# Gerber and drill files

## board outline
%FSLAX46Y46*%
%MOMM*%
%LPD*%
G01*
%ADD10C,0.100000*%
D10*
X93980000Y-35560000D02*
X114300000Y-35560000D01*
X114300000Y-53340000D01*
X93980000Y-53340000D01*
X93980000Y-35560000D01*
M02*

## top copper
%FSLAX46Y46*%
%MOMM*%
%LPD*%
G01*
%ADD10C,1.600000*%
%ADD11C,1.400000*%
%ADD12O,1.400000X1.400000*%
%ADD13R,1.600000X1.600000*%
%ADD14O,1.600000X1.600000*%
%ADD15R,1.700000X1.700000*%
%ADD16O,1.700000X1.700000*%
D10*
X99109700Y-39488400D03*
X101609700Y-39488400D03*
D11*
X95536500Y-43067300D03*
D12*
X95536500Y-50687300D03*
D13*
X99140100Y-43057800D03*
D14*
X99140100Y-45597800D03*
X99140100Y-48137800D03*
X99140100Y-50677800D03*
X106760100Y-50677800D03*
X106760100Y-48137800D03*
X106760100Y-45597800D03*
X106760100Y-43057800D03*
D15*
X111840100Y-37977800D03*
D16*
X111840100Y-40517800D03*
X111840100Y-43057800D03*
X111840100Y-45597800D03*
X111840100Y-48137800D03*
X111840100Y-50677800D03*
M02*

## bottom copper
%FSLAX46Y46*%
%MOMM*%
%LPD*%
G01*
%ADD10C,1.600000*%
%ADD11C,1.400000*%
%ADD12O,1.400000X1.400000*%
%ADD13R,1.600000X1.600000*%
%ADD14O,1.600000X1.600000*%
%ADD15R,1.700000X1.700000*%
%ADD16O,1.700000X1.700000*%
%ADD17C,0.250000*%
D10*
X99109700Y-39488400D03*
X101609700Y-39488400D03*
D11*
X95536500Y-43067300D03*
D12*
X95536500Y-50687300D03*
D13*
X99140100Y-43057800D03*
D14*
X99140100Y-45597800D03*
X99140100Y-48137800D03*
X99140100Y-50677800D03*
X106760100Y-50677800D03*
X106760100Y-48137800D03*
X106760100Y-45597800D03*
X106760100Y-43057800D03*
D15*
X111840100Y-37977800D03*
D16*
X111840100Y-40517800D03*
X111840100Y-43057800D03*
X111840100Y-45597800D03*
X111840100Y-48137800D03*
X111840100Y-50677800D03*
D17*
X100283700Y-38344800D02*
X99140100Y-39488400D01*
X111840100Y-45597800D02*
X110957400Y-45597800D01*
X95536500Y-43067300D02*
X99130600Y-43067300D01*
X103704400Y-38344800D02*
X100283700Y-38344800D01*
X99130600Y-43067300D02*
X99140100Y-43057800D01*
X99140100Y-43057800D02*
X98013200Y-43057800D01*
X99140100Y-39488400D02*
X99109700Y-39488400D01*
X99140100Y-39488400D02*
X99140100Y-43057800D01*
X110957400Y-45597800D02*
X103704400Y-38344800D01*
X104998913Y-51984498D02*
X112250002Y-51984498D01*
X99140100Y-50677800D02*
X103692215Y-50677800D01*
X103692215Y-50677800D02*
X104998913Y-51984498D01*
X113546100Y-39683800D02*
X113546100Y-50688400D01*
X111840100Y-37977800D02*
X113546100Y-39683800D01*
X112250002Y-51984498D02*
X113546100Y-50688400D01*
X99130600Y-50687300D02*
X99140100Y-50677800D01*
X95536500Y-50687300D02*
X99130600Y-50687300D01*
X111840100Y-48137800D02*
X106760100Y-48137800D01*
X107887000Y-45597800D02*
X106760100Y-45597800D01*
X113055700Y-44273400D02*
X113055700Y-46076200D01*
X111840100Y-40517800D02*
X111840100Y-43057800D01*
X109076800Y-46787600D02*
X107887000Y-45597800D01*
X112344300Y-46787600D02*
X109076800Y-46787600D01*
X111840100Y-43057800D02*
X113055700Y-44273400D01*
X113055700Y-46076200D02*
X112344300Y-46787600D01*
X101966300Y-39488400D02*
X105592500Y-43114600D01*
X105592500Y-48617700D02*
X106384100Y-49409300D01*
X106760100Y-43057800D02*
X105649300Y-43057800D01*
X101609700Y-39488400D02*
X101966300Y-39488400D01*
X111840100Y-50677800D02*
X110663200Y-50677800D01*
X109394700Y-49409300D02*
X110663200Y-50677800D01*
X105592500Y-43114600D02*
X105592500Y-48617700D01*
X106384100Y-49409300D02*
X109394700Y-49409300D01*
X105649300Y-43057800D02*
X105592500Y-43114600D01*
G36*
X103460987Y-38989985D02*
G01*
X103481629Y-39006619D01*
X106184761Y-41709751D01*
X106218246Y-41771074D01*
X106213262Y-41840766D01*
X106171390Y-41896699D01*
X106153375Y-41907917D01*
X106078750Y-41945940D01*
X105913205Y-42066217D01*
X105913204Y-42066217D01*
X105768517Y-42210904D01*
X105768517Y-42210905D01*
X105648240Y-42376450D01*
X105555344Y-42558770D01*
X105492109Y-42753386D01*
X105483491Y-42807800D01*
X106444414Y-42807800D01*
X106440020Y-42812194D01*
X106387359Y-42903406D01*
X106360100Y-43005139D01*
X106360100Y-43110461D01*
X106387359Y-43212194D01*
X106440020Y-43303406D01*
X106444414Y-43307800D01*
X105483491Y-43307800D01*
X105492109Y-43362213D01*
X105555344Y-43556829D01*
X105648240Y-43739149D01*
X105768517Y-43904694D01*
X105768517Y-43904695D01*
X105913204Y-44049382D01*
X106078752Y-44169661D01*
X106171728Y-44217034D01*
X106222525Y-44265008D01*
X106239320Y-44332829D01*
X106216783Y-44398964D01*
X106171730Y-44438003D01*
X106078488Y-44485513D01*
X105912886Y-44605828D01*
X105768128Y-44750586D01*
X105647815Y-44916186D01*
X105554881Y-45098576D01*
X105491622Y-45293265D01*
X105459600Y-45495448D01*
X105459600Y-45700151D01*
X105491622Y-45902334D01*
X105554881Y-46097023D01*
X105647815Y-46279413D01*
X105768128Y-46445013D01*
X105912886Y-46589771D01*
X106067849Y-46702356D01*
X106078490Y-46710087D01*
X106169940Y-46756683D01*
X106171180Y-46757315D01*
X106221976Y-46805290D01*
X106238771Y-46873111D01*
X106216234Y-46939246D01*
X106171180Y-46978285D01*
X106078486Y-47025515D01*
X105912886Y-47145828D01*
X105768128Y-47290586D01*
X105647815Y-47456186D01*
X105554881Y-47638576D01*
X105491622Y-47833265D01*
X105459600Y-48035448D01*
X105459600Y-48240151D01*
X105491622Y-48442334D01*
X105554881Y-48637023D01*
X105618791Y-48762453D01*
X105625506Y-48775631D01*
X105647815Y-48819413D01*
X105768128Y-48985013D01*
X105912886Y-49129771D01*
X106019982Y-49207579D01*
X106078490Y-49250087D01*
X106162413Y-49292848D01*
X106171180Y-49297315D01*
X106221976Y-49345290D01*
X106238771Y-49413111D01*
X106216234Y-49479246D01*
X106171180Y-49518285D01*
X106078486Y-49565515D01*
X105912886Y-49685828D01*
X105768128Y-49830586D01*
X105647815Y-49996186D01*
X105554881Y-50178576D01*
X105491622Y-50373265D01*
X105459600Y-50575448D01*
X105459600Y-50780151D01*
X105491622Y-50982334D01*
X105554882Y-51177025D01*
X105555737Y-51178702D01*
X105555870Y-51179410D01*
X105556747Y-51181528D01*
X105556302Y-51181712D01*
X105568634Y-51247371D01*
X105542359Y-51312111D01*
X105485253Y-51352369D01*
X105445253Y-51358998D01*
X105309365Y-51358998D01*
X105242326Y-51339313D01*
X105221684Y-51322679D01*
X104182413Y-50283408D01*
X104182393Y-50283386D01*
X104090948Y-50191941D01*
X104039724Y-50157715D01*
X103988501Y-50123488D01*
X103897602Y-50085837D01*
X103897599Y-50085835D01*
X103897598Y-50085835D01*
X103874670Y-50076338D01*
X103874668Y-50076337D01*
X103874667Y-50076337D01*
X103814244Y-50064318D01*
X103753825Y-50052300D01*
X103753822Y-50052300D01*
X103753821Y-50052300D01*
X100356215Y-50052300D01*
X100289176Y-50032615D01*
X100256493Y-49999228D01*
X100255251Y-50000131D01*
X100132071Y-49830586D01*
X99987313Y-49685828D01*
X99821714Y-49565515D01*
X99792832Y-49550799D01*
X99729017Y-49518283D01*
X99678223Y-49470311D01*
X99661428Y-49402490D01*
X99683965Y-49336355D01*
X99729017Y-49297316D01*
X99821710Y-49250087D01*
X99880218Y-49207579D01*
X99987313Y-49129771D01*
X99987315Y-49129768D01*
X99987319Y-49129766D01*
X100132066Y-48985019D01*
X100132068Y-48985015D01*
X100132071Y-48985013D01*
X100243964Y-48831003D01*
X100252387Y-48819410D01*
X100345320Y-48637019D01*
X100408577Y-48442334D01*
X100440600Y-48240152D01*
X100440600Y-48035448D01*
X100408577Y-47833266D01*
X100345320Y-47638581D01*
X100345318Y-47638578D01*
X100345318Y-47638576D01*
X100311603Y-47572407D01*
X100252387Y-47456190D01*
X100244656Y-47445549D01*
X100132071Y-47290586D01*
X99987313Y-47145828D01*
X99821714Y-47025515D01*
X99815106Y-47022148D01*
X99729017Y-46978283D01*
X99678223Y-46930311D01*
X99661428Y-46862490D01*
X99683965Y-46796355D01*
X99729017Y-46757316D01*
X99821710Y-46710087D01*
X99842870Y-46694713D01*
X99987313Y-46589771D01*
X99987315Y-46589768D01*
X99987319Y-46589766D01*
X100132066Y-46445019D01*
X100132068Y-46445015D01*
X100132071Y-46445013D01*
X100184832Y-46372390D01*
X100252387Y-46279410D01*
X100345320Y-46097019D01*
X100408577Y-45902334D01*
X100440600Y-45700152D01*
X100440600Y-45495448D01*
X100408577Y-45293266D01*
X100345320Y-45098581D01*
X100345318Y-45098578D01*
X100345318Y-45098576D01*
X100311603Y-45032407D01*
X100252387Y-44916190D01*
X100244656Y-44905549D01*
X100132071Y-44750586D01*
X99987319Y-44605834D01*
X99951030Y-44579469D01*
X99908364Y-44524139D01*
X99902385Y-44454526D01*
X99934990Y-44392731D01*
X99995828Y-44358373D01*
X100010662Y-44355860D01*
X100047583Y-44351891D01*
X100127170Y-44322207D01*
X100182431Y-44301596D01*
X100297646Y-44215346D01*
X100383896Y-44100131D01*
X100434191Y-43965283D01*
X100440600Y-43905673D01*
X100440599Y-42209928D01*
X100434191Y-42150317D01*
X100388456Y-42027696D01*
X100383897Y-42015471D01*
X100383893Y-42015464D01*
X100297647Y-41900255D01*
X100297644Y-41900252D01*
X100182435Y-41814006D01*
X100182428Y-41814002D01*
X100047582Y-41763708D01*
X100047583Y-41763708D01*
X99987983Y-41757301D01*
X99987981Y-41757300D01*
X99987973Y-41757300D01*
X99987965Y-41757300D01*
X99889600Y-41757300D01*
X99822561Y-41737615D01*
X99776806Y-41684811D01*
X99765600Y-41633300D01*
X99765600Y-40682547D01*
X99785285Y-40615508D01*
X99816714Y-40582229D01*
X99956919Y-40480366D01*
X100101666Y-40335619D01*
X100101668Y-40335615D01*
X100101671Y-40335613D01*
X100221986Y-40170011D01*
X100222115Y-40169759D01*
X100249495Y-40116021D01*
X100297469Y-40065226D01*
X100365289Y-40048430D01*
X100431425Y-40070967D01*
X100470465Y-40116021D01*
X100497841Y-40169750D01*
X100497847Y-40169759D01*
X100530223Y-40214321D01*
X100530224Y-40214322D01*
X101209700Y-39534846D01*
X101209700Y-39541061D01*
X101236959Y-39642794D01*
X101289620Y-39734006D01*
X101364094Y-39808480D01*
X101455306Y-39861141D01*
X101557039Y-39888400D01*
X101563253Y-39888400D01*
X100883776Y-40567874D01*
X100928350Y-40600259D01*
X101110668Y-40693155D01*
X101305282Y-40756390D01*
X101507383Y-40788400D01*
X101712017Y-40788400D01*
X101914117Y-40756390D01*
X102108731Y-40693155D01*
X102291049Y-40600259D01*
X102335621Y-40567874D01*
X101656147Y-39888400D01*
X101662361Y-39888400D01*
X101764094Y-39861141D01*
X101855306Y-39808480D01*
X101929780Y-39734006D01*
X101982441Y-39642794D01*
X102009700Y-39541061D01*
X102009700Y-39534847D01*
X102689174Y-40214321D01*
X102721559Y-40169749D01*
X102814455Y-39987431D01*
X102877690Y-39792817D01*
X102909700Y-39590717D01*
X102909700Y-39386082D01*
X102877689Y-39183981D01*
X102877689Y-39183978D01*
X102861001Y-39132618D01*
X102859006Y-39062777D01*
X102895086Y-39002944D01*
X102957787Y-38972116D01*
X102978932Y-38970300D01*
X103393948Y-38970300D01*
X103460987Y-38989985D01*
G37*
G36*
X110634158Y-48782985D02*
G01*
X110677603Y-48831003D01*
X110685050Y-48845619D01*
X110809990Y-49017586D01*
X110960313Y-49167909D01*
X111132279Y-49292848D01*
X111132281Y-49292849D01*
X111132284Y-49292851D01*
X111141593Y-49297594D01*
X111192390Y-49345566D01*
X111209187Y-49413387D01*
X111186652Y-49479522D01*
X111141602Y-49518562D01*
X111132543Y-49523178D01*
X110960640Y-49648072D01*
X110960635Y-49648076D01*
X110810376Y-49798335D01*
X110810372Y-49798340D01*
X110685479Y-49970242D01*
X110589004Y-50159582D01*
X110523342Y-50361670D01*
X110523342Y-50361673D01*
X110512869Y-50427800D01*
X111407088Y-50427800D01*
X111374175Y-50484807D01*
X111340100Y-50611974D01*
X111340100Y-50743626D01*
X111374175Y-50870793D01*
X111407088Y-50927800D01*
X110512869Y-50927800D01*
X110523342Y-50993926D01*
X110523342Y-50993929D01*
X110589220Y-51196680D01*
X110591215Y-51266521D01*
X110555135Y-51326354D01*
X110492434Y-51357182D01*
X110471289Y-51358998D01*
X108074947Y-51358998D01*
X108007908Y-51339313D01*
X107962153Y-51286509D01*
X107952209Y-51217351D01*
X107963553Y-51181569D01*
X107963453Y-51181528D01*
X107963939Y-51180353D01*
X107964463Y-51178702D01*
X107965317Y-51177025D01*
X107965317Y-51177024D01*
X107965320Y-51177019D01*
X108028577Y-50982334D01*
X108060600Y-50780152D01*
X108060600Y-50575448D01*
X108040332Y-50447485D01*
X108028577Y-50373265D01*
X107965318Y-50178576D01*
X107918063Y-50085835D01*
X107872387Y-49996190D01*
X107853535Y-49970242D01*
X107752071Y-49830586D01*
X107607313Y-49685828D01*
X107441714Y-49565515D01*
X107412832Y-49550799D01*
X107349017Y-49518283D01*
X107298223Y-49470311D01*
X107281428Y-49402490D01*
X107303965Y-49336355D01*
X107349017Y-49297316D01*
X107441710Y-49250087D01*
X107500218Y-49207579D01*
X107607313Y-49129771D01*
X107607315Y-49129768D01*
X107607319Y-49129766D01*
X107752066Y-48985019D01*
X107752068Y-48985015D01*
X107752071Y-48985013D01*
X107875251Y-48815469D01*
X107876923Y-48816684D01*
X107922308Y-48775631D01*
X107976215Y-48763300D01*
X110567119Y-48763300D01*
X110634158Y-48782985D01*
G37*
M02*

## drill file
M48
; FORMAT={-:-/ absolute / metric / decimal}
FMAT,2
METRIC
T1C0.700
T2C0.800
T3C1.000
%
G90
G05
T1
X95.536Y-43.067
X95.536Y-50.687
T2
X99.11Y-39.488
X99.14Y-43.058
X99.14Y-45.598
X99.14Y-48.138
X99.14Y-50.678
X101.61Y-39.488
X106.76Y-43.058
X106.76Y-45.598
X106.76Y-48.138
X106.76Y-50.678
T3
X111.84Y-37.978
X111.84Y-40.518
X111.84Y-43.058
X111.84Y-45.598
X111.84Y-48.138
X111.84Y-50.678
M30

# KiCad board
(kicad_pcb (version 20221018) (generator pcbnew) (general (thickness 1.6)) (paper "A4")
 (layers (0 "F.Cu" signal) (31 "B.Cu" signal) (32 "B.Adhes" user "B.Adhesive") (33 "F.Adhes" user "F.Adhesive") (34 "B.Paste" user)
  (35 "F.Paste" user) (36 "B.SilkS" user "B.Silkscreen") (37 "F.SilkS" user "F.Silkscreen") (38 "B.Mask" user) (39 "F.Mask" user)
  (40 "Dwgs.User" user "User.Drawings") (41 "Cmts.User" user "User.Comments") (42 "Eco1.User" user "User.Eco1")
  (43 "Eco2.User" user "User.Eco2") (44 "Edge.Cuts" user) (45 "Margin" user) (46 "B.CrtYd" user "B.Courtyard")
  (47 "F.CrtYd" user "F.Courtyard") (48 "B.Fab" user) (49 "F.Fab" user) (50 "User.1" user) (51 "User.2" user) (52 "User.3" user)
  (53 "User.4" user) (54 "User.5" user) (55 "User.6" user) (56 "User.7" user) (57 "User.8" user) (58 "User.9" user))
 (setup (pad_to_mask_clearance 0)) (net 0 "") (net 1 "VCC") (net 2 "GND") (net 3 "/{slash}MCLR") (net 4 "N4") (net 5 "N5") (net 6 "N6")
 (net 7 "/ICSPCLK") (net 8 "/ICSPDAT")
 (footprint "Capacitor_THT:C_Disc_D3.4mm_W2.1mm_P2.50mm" (layer "F.Cu") (at 99.1097 39.4884)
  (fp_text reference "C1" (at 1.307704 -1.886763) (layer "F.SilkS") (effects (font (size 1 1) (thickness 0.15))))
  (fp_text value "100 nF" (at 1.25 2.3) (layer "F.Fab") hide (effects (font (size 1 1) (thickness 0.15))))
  (pad "1" thru_hole circle (at 0 0) (size 1.6 1.6) (drill 0.8) (layers "*.Cu" "*.Mask") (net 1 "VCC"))
  (pad "2" thru_hole circle (at 2.5 0) (size 1.6 1.6) (drill 0.8) (layers "*.Cu" "*.Mask") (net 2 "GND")))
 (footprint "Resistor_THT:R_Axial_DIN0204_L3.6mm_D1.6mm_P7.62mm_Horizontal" (layer "F.Cu") (at 95.5365 43.0673 -90)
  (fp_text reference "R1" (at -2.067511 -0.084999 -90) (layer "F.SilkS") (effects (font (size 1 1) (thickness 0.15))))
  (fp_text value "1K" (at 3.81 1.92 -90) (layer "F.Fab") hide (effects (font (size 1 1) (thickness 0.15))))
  (pad "1" thru_hole circle (at 0 0 270) (size 1.4 1.4) (drill 0.7) (layers "*.Cu" "*.Mask") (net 1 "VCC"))
  (pad "2" thru_hole oval (at 7.62 0 270) (size 1.4 1.4) (drill 0.7) (layers "*.Cu" "*.Mask") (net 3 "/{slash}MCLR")))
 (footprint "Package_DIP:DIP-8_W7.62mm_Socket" (layer "F.Cu") (at 99.1401 43.0578)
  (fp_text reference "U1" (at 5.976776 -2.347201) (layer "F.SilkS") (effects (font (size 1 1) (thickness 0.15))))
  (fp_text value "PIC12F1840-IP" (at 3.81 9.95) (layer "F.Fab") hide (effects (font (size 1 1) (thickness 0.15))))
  (pad "1" thru_hole rect (at 0 0) (size 1.6 1.6) (drill 0.8) (layers "*.Cu" "*.Mask") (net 1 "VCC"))
  (pad "2" thru_hole oval (at 0 2.54) (size 1.6 1.6) (drill 0.8) (layers "*.Cu" "*.Mask") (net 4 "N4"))
  (pad "3" thru_hole oval (at 0 5.08) (size 1.6 1.6) (drill 0.8) (layers "*.Cu" "*.Mask") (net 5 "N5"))
  (pad "4" thru_hole oval (at 0 7.62) (size 1.6 1.6) (drill 0.8) (layers "*.Cu" "*.Mask") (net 3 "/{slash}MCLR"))
  (pad "5" thru_hole oval (at 7.62 7.62) (size 1.6 1.6) (drill 0.8) (layers "*.Cu" "*.Mask") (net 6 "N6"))
  (pad "6" thru_hole oval (at 7.62 5.08) (size 1.6 1.6) (drill 0.8) (layers "*.Cu" "*.Mask") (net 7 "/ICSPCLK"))
  (pad "7" thru_hole oval (at 7.62 2.54) (size 1.6 1.6) (drill 0.8) (layers "*.Cu" "*.Mask") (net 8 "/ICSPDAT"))
  (pad "8" thru_hole oval (at 7.62 0) (size 1.6 1.6) (drill 0.8) (layers "*.Cu" "*.Mask") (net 2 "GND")))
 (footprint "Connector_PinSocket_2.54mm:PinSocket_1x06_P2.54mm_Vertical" (layer "F.Cu") (at 111.8401 37.9778)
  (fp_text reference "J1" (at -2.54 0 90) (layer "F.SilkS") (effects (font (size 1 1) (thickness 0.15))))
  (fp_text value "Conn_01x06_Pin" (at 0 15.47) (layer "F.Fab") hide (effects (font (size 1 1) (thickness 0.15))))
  (pad "1" thru_hole rect (at 0 0) (size 1.7 1.7) (drill 1) (layers "*.Cu" "*.Mask") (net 3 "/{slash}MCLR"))
  (pad "2" thru_hole oval (at 0 2.54) (size 1.7 1.7) (drill 1) (layers "*.Cu" "*.Mask") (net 8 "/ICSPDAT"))
  (pad "3" thru_hole oval (at 0 5.08) (size 1.7 1.7) (drill 1) (layers "*.Cu" "*.Mask") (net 8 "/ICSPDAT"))
  (pad "4" thru_hole oval (at 0 7.62) (size 1.7 1.7) (drill 1) (layers "*.Cu" "*.Mask") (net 1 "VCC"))
  (pad "5" thru_hole oval (at 0 10.16) (size 1.7 1.7) (drill 1) (layers "*.Cu" "*.Mask") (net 7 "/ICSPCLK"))
  (pad "6" thru_hole oval (at 0 12.7) (size 1.7 1.7) (drill 1) (layers "*.Cu" "*.Mask") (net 2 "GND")))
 (gr_rect (start 93.98 35.56) (end 114.3 53.34) (stroke (width 0.1) (type default)) (fill none) (layer "Edge.Cuts"))
 (segment (start 100.2837 38.3448) (end 99.1401 39.4884) (width 0.25) (layer "B.Cu") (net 1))
 (segment (start 111.8401 45.5978) (end 110.9574 45.5978) (width 0.25) (layer "B.Cu") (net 1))
 (segment (start 95.5365 43.0673) (end 99.1306 43.0673) (width 0.25) (layer "B.Cu") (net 1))
 (segment (start 103.7044 38.3448) (end 100.2837 38.3448) (width 0.25) (layer "B.Cu") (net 1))
 (segment (start 99.1306 43.0673) (end 99.1401 43.0578) (width 0.25) (layer "B.Cu") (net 1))
 (segment (start 99.1401 43.0578) (end 98.0132 43.0578) (width 0.25) (layer "B.Cu") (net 1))
 (segment (start 99.1401 39.4884) (end 99.1097 39.4884) (width 0.25) (layer "B.Cu") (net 1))
 (segment (start 99.1401 39.4884) (end 99.1401 43.0578) (width 0.25) (layer "B.Cu") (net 1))
 (segment (start 110.9574 45.5978) (end 103.7044 38.3448) (width 0.25) (layer "B.Cu") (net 1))
 (segment (start 104.998913 51.984498) (end 112.250002 51.984498) (width 0.25) (layer "B.Cu") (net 3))
 (segment (start 99.1401 50.6778) (end 103.692215 50.6778) (width 0.25) (layer "B.Cu") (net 3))
 (segment (start 103.692215 50.6778) (end 104.998913 51.984498) (width 0.25) (layer "B.Cu") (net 3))
 (segment (start 113.5461 39.6838) (end 113.5461 50.6884) (width 0.25) (layer "B.Cu") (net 3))
 (segment (start 111.8401 37.9778) (end 113.5461 39.6838) (width 0.25) (layer "B.Cu") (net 3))
 (segment (start 112.250002 51.984498) (end 113.5461 50.6884) (width 0.25) (layer "B.Cu") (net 3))
 (segment (start 99.1306 50.6873) (end 99.1401 50.6778) (width 0.25) (layer "B.Cu") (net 3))
 (segment (start 95.5365 50.6873) (end 99.1306 50.6873) (width 0.25) (layer "B.Cu") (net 3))
 (segment (start 111.8401 48.1378) (end 106.7601 48.1378) (width 0.25) (layer "B.Cu") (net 7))
 (segment (start 107.887 45.5978) (end 106.7601 45.5978) (width 0.25) (layer "B.Cu") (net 8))
 (segment (start 113.0557 44.2734) (end 113.0557 46.0762) (width 0.25) (layer "B.Cu") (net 8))
 (segment (start 111.8401 40.5178) (end 111.8401 43.0578) (width 0.25) (layer "B.Cu") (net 8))
 (segment (start 109.0768 46.7876) (end 107.887 45.5978) (width 0.25) (layer "B.Cu") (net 8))
 (segment (start 112.3443 46.7876) (end 109.0768 46.7876) (width 0.25) (layer "B.Cu") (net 8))
 (segment (start 111.8401 43.0578) (end 113.0557 44.2734) (width 0.25) (layer "B.Cu") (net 8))
 (segment (start 113.0557 46.0762) (end 112.3443 46.7876) (width 0.25) (layer "B.Cu") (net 8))
 (segment (start 101.9663 39.4884) (end 105.5925 43.1146) (width 0.25) (layer "B.Cu") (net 2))
 (segment (start 105.5925 48.6177) (end 106.3841 49.4093) (width 0.25) (layer "B.Cu") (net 2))
 (segment (start 106.7601 43.0578) (end 105.6493 43.0578) (width 0.25) (layer "B.Cu") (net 2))
 (segment (start 101.6097 39.4884) (end 101.9663 39.4884) (width 0.25) (layer "B.Cu") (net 2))
 (segment (start 111.8401 50.6778) (end 110.6632 50.6778) (width 0.25) (layer "B.Cu") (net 2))
 (segment (start 109.3947 49.4093) (end 110.6632 50.6778) (width 0.25) (layer "B.Cu") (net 2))
 (segment (start 105.5925 43.1146) (end 105.5925 48.6177) (width 0.25) (layer "B.Cu") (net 2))
 (segment (start 106.3841 49.4093) (end 109.3947 49.4093) (width 0.25) (layer "B.Cu") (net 2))
 (segment (start 105.6493 43.0578) (end 105.5925 43.1146) (width 0.25) (layer "B.Cu") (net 2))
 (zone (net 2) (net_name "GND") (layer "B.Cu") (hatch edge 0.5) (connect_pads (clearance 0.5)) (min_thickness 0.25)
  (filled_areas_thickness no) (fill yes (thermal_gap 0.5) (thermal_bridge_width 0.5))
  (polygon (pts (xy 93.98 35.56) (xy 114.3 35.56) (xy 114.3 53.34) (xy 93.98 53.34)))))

